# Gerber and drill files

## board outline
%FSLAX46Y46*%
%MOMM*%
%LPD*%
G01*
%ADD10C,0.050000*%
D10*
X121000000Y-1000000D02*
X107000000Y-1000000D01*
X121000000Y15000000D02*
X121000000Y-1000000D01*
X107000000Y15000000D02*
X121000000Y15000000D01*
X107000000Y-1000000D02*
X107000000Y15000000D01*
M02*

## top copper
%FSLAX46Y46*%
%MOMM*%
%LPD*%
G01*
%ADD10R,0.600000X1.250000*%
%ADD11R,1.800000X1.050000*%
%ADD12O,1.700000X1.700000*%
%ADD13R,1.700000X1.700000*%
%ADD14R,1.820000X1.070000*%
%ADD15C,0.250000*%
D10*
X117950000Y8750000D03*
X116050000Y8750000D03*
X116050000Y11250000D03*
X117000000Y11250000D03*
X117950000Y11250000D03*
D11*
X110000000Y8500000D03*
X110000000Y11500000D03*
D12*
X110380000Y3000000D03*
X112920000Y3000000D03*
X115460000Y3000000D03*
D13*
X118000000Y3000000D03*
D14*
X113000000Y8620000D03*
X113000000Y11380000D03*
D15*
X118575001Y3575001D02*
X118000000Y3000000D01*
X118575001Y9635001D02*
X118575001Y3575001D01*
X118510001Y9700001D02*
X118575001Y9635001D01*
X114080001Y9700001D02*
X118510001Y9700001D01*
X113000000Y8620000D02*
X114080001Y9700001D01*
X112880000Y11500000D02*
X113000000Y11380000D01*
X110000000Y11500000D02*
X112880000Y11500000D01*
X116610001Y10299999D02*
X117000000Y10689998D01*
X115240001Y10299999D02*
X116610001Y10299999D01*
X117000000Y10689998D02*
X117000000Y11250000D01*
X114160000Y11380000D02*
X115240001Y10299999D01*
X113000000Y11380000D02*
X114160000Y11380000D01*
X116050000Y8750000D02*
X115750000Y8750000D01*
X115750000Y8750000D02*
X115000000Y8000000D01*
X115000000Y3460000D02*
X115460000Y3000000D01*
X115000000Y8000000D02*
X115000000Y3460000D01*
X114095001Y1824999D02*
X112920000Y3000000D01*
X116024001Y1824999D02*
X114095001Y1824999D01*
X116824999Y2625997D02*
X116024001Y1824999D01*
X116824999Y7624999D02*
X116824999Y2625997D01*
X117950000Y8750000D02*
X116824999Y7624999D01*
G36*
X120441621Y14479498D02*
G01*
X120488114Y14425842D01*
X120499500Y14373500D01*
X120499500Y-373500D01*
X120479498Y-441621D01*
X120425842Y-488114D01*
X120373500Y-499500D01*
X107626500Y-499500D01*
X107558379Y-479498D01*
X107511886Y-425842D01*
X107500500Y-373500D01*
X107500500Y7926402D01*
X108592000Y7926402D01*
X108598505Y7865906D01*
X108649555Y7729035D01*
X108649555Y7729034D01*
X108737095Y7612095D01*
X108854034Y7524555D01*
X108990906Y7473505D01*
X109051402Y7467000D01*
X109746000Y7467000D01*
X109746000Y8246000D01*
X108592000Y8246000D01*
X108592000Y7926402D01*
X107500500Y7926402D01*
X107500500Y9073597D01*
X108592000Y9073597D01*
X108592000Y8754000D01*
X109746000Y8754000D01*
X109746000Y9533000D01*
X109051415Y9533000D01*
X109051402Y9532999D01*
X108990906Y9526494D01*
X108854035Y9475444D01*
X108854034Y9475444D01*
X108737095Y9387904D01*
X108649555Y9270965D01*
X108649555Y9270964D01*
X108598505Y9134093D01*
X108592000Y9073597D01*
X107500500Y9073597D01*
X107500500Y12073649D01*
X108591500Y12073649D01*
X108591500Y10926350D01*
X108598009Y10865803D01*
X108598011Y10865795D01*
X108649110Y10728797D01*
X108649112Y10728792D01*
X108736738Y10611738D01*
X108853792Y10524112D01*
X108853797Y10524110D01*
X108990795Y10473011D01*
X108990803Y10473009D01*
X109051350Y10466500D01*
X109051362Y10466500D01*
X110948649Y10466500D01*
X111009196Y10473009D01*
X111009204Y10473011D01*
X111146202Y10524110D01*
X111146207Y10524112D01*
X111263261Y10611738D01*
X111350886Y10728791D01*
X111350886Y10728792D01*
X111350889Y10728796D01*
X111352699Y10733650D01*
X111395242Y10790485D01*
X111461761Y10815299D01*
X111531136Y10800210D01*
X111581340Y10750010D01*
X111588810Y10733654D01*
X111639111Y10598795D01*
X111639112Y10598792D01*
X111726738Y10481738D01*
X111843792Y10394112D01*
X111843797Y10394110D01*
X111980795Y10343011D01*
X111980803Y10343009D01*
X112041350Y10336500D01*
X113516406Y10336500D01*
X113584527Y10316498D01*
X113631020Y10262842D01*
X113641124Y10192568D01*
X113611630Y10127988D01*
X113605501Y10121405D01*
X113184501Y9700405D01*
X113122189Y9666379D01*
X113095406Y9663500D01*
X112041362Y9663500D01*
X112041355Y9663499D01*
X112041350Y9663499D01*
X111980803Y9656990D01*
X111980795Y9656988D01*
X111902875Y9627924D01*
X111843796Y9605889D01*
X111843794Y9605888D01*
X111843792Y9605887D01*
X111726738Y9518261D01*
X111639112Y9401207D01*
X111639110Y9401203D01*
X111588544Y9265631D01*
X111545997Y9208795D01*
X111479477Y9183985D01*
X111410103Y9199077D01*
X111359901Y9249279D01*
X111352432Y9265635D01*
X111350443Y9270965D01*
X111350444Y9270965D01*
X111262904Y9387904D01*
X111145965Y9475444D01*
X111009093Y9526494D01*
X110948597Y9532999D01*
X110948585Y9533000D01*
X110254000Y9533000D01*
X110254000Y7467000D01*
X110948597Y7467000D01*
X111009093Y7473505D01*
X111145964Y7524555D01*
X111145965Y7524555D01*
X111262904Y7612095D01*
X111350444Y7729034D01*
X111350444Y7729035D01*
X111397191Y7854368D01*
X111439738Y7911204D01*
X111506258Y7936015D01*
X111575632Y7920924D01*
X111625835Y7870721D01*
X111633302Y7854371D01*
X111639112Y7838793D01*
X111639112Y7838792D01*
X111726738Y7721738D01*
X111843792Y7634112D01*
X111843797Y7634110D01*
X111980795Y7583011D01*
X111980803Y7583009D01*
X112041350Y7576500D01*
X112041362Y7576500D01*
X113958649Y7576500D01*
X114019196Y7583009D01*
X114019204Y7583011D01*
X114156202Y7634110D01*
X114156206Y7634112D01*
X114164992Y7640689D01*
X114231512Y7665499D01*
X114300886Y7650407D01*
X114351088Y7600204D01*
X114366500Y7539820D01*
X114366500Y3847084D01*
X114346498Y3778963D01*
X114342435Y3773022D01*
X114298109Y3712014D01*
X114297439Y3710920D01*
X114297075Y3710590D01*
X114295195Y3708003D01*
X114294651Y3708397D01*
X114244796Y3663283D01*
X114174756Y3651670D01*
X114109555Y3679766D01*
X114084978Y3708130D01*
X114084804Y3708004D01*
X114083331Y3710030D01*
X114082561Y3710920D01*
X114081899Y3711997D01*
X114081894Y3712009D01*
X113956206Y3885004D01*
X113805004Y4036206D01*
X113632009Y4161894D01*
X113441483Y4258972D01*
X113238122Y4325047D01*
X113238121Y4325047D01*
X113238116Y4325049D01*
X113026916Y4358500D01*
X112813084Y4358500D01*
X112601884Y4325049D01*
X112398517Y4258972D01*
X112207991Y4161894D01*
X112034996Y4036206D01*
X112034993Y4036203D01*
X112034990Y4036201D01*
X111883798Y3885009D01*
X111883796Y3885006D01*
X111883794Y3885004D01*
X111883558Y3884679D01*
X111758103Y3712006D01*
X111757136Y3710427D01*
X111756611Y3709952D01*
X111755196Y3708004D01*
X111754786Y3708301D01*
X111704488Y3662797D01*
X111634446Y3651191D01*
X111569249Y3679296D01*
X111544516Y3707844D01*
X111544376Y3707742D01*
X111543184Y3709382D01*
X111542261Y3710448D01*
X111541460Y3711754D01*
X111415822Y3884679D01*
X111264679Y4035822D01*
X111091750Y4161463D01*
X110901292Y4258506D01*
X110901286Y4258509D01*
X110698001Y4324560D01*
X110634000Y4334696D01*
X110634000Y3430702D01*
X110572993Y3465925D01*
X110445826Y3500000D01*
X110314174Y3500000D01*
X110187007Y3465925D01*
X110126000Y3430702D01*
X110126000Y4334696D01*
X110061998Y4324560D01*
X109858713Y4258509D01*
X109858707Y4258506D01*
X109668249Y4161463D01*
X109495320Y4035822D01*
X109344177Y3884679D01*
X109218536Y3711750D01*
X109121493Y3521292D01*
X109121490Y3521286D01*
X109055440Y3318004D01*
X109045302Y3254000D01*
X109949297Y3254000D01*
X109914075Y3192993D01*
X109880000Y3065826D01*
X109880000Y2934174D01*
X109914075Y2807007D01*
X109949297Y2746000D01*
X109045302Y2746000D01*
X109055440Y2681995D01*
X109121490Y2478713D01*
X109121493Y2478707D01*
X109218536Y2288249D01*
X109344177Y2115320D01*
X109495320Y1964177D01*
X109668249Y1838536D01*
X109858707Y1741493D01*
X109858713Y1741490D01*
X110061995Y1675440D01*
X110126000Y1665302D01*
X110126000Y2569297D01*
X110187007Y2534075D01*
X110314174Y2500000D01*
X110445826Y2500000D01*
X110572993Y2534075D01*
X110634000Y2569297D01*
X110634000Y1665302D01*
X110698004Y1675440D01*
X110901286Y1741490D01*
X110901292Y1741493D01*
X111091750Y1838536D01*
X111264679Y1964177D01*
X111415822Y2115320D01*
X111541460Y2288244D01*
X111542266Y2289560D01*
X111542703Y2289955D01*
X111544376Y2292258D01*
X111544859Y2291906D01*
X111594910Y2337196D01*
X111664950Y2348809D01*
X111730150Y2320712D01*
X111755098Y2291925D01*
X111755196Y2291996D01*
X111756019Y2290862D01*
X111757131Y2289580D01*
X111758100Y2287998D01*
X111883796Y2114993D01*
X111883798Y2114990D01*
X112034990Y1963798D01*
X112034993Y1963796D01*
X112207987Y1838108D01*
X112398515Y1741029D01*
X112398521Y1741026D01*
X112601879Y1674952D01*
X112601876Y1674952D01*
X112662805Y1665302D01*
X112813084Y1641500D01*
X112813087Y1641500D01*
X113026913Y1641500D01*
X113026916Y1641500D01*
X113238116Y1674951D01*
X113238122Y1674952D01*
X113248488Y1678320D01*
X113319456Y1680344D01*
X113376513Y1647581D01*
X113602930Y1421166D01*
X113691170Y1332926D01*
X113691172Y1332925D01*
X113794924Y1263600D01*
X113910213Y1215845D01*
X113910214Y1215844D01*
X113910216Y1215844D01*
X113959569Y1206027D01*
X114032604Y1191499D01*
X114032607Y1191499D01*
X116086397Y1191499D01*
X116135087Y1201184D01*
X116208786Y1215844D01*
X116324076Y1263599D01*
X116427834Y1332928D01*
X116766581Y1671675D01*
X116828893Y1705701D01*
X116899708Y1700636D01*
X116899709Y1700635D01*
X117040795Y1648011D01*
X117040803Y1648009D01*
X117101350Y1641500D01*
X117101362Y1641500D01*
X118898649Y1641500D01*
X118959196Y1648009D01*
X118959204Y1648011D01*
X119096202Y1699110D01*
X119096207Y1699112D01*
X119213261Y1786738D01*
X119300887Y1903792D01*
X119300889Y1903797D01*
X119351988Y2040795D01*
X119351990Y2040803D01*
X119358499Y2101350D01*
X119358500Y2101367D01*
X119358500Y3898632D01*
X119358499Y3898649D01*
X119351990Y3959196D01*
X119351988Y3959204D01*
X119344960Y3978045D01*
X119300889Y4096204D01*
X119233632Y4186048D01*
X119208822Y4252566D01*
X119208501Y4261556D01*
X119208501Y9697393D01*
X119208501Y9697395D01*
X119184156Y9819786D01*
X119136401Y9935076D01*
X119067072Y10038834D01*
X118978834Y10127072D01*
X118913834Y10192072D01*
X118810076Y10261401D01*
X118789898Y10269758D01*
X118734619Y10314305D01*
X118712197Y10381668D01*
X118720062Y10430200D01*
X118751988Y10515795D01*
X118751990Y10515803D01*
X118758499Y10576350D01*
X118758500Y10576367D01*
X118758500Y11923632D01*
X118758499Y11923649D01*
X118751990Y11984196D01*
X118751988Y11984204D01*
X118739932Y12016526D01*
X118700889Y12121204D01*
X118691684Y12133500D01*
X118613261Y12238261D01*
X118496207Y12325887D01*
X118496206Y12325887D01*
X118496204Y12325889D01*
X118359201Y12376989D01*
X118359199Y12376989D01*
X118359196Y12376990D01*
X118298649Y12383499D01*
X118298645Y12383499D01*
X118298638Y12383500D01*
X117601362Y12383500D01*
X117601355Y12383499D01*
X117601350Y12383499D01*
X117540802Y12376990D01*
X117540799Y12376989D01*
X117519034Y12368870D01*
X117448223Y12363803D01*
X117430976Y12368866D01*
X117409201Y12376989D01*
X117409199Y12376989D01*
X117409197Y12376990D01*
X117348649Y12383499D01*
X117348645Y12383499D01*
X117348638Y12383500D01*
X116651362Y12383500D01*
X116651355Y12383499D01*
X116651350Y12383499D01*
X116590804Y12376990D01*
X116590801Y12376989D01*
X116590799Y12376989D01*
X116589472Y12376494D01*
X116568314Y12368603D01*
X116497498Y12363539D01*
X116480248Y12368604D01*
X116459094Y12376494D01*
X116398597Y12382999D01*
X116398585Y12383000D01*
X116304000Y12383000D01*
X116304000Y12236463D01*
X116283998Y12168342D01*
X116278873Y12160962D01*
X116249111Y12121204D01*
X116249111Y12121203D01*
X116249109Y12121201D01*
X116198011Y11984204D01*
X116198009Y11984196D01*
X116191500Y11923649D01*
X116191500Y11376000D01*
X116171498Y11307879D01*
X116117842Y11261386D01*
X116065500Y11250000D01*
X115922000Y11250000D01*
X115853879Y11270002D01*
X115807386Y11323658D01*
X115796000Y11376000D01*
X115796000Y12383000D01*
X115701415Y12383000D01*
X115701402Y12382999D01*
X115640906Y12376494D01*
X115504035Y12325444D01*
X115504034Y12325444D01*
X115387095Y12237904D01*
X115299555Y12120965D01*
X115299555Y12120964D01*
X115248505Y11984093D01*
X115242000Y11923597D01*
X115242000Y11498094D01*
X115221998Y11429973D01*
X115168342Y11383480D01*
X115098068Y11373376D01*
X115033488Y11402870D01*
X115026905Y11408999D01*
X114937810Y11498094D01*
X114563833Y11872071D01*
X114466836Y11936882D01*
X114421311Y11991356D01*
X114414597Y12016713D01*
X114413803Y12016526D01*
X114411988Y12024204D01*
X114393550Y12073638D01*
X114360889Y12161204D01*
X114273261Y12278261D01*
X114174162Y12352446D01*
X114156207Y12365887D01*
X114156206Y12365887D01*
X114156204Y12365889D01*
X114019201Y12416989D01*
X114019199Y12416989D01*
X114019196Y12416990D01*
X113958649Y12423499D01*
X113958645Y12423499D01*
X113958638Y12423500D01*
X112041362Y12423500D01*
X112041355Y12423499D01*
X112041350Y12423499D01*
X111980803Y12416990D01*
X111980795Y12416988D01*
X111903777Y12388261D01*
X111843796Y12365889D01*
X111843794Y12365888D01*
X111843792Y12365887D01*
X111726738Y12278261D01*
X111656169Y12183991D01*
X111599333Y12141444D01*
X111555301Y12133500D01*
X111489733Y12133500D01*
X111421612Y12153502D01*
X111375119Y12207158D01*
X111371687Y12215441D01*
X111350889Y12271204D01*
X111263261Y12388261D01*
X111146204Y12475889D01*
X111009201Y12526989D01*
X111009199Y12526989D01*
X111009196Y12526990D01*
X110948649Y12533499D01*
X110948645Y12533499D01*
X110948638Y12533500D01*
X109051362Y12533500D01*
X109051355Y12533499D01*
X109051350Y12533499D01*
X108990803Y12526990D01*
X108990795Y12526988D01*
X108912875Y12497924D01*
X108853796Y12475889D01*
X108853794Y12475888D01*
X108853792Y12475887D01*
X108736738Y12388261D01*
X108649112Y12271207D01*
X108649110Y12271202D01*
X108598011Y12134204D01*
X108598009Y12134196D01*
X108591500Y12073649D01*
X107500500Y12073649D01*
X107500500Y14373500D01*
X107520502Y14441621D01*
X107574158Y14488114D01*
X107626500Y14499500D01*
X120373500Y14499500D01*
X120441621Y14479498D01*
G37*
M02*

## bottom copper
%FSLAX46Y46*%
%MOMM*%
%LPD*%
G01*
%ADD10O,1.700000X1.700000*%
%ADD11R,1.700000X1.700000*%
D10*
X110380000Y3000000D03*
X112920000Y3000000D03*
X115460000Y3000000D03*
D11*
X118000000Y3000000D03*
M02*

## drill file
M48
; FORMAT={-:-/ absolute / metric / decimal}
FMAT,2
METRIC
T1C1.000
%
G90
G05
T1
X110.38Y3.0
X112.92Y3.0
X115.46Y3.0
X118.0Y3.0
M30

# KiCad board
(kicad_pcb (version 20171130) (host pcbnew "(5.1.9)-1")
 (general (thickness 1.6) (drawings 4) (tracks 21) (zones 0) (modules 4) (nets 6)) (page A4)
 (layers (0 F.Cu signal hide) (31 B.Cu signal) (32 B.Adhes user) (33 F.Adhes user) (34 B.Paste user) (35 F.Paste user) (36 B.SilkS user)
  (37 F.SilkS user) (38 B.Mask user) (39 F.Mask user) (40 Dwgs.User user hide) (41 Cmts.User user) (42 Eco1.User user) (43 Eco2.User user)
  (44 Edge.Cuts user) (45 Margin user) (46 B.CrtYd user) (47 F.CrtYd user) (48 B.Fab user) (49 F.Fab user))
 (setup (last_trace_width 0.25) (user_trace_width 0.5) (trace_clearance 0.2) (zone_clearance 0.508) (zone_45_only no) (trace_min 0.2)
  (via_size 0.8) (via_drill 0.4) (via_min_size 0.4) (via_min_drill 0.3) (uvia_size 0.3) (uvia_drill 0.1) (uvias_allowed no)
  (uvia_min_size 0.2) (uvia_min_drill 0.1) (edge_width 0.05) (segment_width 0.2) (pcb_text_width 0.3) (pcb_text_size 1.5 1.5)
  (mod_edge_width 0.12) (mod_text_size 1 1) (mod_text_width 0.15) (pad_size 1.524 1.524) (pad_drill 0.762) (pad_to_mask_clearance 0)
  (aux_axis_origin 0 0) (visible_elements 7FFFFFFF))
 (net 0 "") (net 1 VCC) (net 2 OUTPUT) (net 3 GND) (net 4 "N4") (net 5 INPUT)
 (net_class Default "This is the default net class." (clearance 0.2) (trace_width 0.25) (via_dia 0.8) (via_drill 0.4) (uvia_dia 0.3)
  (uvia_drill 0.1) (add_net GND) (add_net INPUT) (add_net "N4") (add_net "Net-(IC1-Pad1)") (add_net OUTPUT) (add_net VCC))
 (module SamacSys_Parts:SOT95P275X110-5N (layer F.Cu) (at 117 -10 270)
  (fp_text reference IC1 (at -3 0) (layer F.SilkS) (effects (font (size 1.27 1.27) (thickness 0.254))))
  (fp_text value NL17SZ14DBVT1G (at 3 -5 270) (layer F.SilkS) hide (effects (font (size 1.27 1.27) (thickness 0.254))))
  (pad 5 smd rect (at 1.25 -0.95) (size 0.6 1.25) (layers F.Cu F.Paste F.Mask) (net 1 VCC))
  (pad 4 smd rect (at 1.25 0.95) (size 0.6 1.25) (layers F.Cu F.Paste F.Mask) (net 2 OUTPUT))
  (pad 3 smd rect (at -1.25 0.95) (size 0.6 1.25) (layers F.Cu F.Paste F.Mask) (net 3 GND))
  (pad 2 smd rect (at -1.25 0) (size 0.6 1.25) (layers F.Cu F.Paste F.Mask) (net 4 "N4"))
  (pad 1 smd rect (at -1.25 -0.95) (size 0.6 1.25) (layers F.Cu F.Paste F.Mask)))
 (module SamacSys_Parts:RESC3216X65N (layer F.Cu) (at 110 -10 270)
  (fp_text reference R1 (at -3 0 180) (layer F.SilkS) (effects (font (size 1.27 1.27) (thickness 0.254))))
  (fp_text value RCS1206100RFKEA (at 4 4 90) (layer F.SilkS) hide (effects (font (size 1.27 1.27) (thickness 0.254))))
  (pad 2 smd rect (at 1.5 0 270) (size 1.05 1.8) (layers F.Cu F.Paste F.Mask) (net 3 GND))
  (pad 1 smd rect (at -1.5 0 270) (size 1.05 1.8) (layers F.Cu F.Paste F.Mask) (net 4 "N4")))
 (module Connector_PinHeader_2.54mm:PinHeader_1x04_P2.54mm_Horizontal (layer F.Cu) (at 118 -3 270)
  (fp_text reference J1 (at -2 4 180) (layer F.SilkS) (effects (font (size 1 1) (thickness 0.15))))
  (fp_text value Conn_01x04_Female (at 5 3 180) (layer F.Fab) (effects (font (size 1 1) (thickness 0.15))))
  (pad 4 thru_hole oval (at 0 7.62 270) (size 1.7 1.7) (drill 1) (layers *.Cu *.Mask) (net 3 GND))
  (pad 3 thru_hole oval (at 0 5.08 270) (size 1.7 1.7) (drill 1) (layers *.Cu *.Mask) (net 1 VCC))
  (pad 2 thru_hole oval (at 0 2.54 270) (size 1.7 1.7) (drill 1) (layers *.Cu *.Mask) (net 2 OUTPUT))
  (pad 1 thru_hole rect (at 0 0 270) (size 1.7 1.7) (drill 1) (layers *.Cu *.Mask) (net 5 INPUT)))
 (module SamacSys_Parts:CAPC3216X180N (layer F.Cu) (at 113 -10 270)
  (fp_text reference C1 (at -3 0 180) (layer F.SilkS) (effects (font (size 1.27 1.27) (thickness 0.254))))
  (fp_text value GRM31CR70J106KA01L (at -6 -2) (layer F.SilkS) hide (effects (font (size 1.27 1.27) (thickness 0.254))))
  (pad 2 smd rect (at 1.38 0 270) (size 1.07 1.82) (layers F.Cu F.Paste F.Mask) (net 5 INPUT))
  (pad 1 smd rect (at -1.38 0 270) (size 1.07 1.82) (layers F.Cu F.Paste F.Mask) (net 4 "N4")))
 (gr_line (start 121 1) (end 107 1) (layer Edge.Cuts) (width 0.05))
 (gr_line (start 121 -15) (end 121 1) (layer Edge.Cuts) (width 0.05))
 (gr_line (start 107 -15) (end 121 -15) (layer Edge.Cuts) (width 0.05))
 (gr_line (start 107 1) (end 107 -15) (layer Edge.Cuts) (width 0.05))
 (segment (start 118.575001 -3.575001) (end 118 -3) (width 0.25) (layer F.Cu) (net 5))
 (segment (start 118.575001 -9.635001) (end 118.575001 -3.575001) (width 0.25) (layer F.Cu) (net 5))
 (segment (start 118.510001 -9.700001) (end 118.575001 -9.635001) (width 0.25) (layer F.Cu) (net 5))
 (segment (start 114.080001 -9.700001) (end 118.510001 -9.700001) (width 0.25) (layer F.Cu) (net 5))
 (segment (start 113 -8.62) (end 114.080001 -9.700001) (width 0.25) (layer F.Cu) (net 5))
 (segment (start 112.88 -11.5) (end 113 -11.38) (width 0.25) (layer F.Cu) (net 4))
 (segment (start 110 -11.5) (end 112.88 -11.5) (width 0.25) (layer F.Cu) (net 4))
 (segment (start 116.610001 -10.299999) (end 117 -10.689998) (width 0.25) (layer F.Cu) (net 4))
 (segment (start 115.240001 -10.299999) (end 116.610001 -10.299999) (width 0.25) (layer F.Cu) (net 4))
 (segment (start 117 -10.689998) (end 117 -11.25) (width 0.25) (layer F.Cu) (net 4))
 (segment (start 114.16 -11.38) (end 115.240001 -10.299999) (width 0.25) (layer F.Cu) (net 4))
 (segment (start 113 -11.38) (end 114.16 -11.38) (width 0.25) (layer F.Cu) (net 4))
 (segment (start 116.05 -8.75) (end 115.75 -8.75) (width 0.25) (layer F.Cu) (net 2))
 (segment (start 115.75 -8.75) (end 115 -8) (width 0.25) (layer F.Cu) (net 2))
 (segment (start 115 -3.46) (end 115.46 -3) (width 0.25) (layer F.Cu) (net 2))
 (segment (start 115 -8) (end 115 -3.46) (width 0.25) (layer F.Cu) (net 2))
 (segment (start 114.095001 -1.824999) (end 112.92 -3) (width 0.25) (layer F.Cu) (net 1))
 (segment (start 116.024001 -1.824999) (end 114.095001 -1.824999) (width 0.25) (layer F.Cu) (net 1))
 (segment (start 116.824999 -2.625997) (end 116.024001 -1.824999) (width 0.25) (layer F.Cu) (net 1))
 (segment (start 116.824999 -7.624999) (end 116.824999 -2.625997) (width 0.25) (layer F.Cu) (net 1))
 (segment (start 117.95 -8.75) (end 116.824999 -7.624999) (width 0.25) (layer F.Cu) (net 1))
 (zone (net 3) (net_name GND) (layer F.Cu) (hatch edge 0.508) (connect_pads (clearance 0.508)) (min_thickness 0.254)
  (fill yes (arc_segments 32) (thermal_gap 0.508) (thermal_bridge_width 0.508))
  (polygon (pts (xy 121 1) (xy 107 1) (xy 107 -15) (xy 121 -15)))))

